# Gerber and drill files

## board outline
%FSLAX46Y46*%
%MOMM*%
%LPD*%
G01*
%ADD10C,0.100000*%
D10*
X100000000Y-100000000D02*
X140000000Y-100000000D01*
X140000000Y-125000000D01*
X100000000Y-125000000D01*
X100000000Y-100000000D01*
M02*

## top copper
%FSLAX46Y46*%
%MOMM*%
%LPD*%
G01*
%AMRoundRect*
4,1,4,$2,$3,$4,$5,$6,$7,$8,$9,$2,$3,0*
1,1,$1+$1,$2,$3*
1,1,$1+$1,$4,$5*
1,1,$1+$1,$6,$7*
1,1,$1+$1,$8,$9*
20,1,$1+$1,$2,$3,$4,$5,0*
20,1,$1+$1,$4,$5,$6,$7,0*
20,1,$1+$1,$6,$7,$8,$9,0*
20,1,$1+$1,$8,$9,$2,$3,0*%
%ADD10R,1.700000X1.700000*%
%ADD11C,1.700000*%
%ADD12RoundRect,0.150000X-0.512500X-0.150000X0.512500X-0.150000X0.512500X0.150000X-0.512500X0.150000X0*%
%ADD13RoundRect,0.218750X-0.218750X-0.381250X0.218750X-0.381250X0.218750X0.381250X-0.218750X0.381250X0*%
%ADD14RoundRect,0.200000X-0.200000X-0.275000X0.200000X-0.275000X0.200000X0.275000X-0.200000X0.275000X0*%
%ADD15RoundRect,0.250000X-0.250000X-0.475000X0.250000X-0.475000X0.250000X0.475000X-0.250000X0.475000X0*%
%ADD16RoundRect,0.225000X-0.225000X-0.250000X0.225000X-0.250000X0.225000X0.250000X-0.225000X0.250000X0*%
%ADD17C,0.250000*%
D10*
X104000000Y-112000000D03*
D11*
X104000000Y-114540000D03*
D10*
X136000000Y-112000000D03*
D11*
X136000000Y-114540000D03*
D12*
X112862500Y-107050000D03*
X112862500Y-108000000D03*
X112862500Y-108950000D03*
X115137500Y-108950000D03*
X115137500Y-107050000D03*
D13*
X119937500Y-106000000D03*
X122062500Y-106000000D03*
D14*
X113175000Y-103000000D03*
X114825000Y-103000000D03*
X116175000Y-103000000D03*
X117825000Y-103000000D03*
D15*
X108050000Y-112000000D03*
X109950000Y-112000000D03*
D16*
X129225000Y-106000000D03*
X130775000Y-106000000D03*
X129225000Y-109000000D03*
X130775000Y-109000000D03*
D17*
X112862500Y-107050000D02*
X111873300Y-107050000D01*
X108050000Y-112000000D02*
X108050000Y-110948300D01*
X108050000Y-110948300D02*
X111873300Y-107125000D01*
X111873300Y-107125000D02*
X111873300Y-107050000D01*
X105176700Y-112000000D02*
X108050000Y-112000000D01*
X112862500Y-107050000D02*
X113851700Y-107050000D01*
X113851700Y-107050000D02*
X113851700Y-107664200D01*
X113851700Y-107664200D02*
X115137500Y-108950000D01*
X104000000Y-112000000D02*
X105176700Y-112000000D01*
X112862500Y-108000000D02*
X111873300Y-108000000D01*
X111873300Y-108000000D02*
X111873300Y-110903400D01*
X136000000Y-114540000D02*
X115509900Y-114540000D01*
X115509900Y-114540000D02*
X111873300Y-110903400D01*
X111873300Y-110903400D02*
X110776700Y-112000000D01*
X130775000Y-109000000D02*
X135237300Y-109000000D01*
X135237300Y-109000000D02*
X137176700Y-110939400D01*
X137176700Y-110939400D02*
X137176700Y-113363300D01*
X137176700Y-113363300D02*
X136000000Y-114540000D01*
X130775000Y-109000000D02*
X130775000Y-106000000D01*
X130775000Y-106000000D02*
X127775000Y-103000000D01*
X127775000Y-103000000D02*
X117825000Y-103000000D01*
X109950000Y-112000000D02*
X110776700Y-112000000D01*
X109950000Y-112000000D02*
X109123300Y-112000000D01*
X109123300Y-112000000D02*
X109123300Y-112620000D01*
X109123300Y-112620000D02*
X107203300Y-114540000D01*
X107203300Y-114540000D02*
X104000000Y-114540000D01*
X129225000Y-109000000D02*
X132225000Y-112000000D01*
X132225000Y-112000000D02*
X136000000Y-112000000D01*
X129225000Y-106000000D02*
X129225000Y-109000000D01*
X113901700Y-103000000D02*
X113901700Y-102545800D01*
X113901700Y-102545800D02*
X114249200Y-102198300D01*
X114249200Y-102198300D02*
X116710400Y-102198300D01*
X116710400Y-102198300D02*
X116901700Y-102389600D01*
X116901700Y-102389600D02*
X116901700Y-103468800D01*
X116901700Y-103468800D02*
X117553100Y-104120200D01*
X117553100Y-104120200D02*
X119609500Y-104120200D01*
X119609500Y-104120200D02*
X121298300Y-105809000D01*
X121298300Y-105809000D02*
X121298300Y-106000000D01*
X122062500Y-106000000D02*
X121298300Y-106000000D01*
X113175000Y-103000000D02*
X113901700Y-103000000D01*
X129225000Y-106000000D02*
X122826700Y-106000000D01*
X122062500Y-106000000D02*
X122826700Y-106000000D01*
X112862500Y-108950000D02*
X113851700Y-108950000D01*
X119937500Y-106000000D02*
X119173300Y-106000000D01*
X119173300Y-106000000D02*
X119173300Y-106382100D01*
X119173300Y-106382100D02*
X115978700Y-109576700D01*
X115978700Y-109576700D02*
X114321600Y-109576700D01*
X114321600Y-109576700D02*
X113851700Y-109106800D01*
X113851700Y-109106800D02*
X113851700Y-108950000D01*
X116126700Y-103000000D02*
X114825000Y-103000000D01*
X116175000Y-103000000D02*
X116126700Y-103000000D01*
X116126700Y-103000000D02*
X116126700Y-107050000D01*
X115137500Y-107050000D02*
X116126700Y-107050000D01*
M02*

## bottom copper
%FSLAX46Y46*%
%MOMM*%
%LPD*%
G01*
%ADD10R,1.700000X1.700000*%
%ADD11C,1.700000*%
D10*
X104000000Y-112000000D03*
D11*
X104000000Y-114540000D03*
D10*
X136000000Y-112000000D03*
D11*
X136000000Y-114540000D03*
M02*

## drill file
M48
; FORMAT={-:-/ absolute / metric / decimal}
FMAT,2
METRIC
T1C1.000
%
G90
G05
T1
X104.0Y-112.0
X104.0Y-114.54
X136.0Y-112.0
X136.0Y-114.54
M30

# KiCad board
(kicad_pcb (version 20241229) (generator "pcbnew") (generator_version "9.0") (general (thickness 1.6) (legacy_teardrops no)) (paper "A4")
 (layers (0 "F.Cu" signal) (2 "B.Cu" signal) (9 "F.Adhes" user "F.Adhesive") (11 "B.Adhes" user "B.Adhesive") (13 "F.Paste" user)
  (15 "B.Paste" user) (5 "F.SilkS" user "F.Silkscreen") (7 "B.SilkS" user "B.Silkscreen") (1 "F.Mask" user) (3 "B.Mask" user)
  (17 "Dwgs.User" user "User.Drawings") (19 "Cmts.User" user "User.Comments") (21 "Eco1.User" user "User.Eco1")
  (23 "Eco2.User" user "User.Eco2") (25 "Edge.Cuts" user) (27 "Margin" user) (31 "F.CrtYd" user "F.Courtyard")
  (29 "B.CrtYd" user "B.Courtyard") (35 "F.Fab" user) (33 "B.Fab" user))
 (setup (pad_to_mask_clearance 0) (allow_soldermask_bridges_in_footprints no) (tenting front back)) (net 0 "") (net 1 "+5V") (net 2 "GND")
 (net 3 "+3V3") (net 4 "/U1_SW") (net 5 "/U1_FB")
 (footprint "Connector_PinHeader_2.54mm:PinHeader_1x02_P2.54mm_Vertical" (layer "F.Cu") (at 104 112)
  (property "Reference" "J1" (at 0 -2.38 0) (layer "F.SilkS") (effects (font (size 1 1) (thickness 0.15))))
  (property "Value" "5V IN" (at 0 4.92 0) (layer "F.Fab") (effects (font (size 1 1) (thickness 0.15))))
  (pad "1" thru_hole rect (at 0 0) (size 1.7 1.7) (drill 1) (layers "*.Cu" "*.Mask") (remove_unused_layers no) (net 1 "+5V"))
  (pad "2" thru_hole circle (at 0 2.54) (size 1.7 1.7) (drill 1) (layers "*.Cu" "*.Mask") (remove_unused_layers no) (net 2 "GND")))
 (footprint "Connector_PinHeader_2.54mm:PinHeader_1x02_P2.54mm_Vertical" (layer "F.Cu") (at 136 112)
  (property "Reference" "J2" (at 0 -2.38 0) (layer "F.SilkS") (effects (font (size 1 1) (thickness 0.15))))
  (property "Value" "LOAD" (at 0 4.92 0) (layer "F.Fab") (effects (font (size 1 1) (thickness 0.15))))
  (pad "1" thru_hole rect (at 0 0) (size 1.7 1.7) (drill 1) (layers "*.Cu" "*.Mask") (remove_unused_layers no) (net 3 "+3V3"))
  (pad "2" thru_hole circle (at 0 2.54) (size 1.7 1.7) (drill 1) (layers "*.Cu" "*.Mask") (remove_unused_layers no) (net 2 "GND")))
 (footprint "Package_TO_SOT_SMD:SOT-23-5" (layer "F.Cu") (at 114 108)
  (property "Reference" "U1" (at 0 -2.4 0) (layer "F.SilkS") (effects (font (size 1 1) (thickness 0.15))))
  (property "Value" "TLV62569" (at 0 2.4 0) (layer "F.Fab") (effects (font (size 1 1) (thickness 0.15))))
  (pad "1" smd roundrect (at -1.1375 -0.95) (size 1.325 0.6) (layers "F.Cu" "F.Mask" "F.Paste") (roundrect_rratio 0.25) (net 1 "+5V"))
  (pad "2" smd roundrect (at -1.1375 0) (size 1.325 0.6) (layers "F.Cu" "F.Mask" "F.Paste") (roundrect_rratio 0.25) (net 2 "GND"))
  (pad "3" smd roundrect (at -1.1375 0.95) (size 1.325 0.6) (layers "F.Cu" "F.Mask" "F.Paste") (roundrect_rratio 0.25) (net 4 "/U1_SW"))
  (pad "4" smd roundrect (at 1.1375 0.95) (size 1.325 0.6) (layers "F.Cu" "F.Mask" "F.Paste") (roundrect_rratio 0.25) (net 1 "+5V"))
  (pad "5" smd roundrect (at 1.1375 -0.95) (size 1.325 0.6) (layers "F.Cu" "F.Mask" "F.Paste") (roundrect_rratio 0.25) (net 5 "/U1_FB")))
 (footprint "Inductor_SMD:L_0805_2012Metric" (layer "F.Cu") (at 121 106)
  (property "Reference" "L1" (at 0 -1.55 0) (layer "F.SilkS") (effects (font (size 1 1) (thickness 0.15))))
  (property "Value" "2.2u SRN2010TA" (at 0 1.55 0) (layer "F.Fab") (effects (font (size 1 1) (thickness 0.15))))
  (pad "1" smd roundrect (at -1.0625 0) (size 0.875 1.2) (layers "F.Cu" "F.Mask" "F.Paste") (roundrect_rratio 0.25) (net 4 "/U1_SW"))
  (pad "2" smd roundrect (at 1.0625 0) (size 0.875 1.2) (layers "F.Cu" "F.Mask" "F.Paste") (roundrect_rratio 0.25) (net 3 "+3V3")))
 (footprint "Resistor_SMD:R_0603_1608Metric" (layer "F.Cu") (at 114 103)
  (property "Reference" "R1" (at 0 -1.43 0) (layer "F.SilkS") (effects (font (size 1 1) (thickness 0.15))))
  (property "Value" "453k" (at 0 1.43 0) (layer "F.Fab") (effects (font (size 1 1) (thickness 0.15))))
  (pad "1" smd roundrect (at -0.825 0) (size 0.8 0.95) (layers "F.Cu" "F.Mask" "F.Paste") (roundrect_rratio 0.25) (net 3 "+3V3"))
  (pad "2" smd roundrect (at 0.825 0) (size 0.8 0.95) (layers "F.Cu" "F.Mask" "F.Paste") (roundrect_rratio 0.25) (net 5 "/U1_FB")))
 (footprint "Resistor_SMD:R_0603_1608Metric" (layer "F.Cu") (at 117 103)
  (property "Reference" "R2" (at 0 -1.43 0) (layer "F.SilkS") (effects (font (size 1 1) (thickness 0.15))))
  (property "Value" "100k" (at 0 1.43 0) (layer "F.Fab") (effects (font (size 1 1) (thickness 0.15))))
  (pad "1" smd roundrect (at -0.825 0) (size 0.8 0.95) (layers "F.Cu" "F.Mask" "F.Paste") (roundrect_rratio 0.25) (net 5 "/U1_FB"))
  (pad "2" smd roundrect (at 0.825 0) (size 0.8 0.95) (layers "F.Cu" "F.Mask" "F.Paste") (roundrect_rratio 0.25) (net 2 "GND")))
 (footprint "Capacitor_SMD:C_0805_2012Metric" (layer "F.Cu") (at 109 112)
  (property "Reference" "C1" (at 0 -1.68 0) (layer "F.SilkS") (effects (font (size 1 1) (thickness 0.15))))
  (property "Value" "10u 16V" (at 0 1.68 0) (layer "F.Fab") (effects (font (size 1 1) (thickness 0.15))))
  (pad "1" smd roundrect (at -0.95 0) (size 1 1.45) (layers "F.Cu" "F.Mask" "F.Paste") (roundrect_rratio 0.25) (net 1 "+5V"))
  (pad "2" smd roundrect (at 0.95 0) (size 1 1.45) (layers "F.Cu" "F.Mask" "F.Paste") (roundrect_rratio 0.25) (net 2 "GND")))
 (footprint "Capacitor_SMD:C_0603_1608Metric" (layer "F.Cu") (at 130 106)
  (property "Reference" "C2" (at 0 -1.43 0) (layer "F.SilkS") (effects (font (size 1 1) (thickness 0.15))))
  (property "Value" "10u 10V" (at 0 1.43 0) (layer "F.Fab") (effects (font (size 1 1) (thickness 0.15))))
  (pad "1" smd roundrect (at -0.775 0) (size 0.9 0.95) (layers "F.Cu" "F.Mask" "F.Paste") (roundrect_rratio 0.25) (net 3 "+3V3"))
  (pad "2" smd roundrect (at 0.775 0) (size 0.9 0.95) (layers "F.Cu" "F.Mask" "F.Paste") (roundrect_rratio 0.25) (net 2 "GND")))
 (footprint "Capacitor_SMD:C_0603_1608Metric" (layer "F.Cu") (at 130 109)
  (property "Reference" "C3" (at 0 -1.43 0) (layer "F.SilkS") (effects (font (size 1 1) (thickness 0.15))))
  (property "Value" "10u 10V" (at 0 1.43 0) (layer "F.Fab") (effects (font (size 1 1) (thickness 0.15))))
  (pad "1" smd roundrect (at -0.775 0) (size 0.9 0.95) (layers "F.Cu" "F.Mask" "F.Paste") (roundrect_rratio 0.25) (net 3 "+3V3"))
  (pad "2" smd roundrect (at 0.775 0) (size 0.9 0.95) (layers "F.Cu" "F.Mask" "F.Paste") (roundrect_rratio 0.25) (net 2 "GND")))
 (gr_rect (start 100 100) (end 140 125) (stroke (width 0.1) (type default)) (fill no) (layer "Edge.Cuts"))
 (segment (start 112.8625 107.05) (end 111.8733 107.05) (width 0.25) (layer "F.Cu") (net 1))
 (segment (start 108.05 112) (end 108.05 110.9483) (width 0.25) (layer "F.Cu") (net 1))
 (segment (start 108.05 110.9483) (end 111.8733 107.125) (width 0.25) (layer "F.Cu") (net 1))
 (segment (start 111.8733 107.125) (end 111.8733 107.05) (width 0.25) (layer "F.Cu") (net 1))
 (segment (start 105.1767 112) (end 108.05 112) (width 0.25) (layer "F.Cu") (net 1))
 (segment (start 112.8625 107.05) (end 113.8517 107.05) (width 0.25) (layer "F.Cu") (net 1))
 (segment (start 113.8517 107.05) (end 113.8517 107.6642) (width 0.25) (layer "F.Cu") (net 1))
 (segment (start 113.8517 107.6642) (end 115.1375 108.95) (width 0.25) (layer "F.Cu") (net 1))
 (segment (start 104 112) (end 105.1767 112) (width 0.25) (layer "F.Cu") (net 1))
 (segment (start 112.8625 108) (end 111.8733 108) (width 0.25) (layer "F.Cu") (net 2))
 (segment (start 111.8733 108) (end 111.8733 110.9034) (width 0.25) (layer "F.Cu") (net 2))
 (segment (start 136 114.54) (end 115.5099 114.54) (width 0.25) (layer "F.Cu") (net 2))
 (segment (start 115.5099 114.54) (end 111.8733 110.9034) (width 0.25) (layer "F.Cu") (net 2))
 (segment (start 111.8733 110.9034) (end 110.7767 112) (width 0.25) (layer "F.Cu") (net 2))
 (segment (start 130.775 109) (end 135.2373 109) (width 0.25) (layer "F.Cu") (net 2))
 (segment (start 135.2373 109) (end 137.1767 110.9394) (width 0.25) (layer "F.Cu") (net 2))
 (segment (start 137.1767 110.9394) (end 137.1767 113.3633) (width 0.25) (layer "F.Cu") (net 2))
 (segment (start 137.1767 113.3633) (end 136 114.54) (width 0.25) (layer "F.Cu") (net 2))
 (segment (start 130.775 109) (end 130.775 106) (width 0.25) (layer "F.Cu") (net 2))
 (segment (start 130.775 106) (end 127.775 103) (width 0.25) (layer "F.Cu") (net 2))
 (segment (start 127.775 103) (end 117.825 103) (width 0.25) (layer "F.Cu") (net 2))
 (segment (start 109.95 112) (end 110.7767 112) (width 0.25) (layer "F.Cu") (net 2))
 (segment (start 109.95 112) (end 109.1233 112) (width 0.25) (layer "F.Cu") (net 2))
 (segment (start 109.1233 112) (end 109.1233 112.62) (width 0.25) (layer "F.Cu") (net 2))
 (segment (start 109.1233 112.62) (end 107.2033 114.54) (width 0.25) (layer "F.Cu") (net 2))
 (segment (start 107.2033 114.54) (end 104 114.54) (width 0.25) (layer "F.Cu") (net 2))
 (segment (start 129.225 109) (end 132.225 112) (width 0.25) (layer "F.Cu") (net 3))
 (segment (start 132.225 112) (end 136 112) (width 0.25) (layer "F.Cu") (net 3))
 (segment (start 129.225 106) (end 129.225 109) (width 0.25) (layer "F.Cu") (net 3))
 (segment (start 113.9017 103) (end 113.9017 102.5458) (width 0.25) (layer "F.Cu") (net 3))
 (segment (start 113.9017 102.5458) (end 114.2492 102.1983) (width 0.25) (layer "F.Cu") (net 3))
 (segment (start 114.2492 102.1983) (end 116.7104 102.1983) (width 0.25) (layer "F.Cu") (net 3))
 (segment (start 116.7104 102.1983) (end 116.9017 102.3896) (width 0.25) (layer "F.Cu") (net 3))
 (segment (start 116.9017 102.3896) (end 116.9017 103.4688) (width 0.25) (layer "F.Cu") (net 3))
 (segment (start 116.9017 103.4688) (end 117.5531 104.1202) (width 0.25) (layer "F.Cu") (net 3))
 (segment (start 117.5531 104.1202) (end 119.6095 104.1202) (width 0.25) (layer "F.Cu") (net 3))
 (segment (start 119.6095 104.1202) (end 121.2983 105.809) (width 0.25) (layer "F.Cu") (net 3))
 (segment (start 121.2983 105.809) (end 121.2983 106) (width 0.25) (layer "F.Cu") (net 3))
 (segment (start 122.0625 106) (end 121.2983 106) (width 0.25) (layer "F.Cu") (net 3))
 (segment (start 113.175 103) (end 113.9017 103) (width 0.25) (layer "F.Cu") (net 3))
 (segment (start 129.225 106) (end 122.8267 106) (width 0.25) (layer "F.Cu") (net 3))
 (segment (start 122.0625 106) (end 122.8267 106) (width 0.25) (layer "F.Cu") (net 3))
 (segment (start 112.8625 108.95) (end 113.8517 108.95) (width 0.25) (layer "F.Cu") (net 4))
 (segment (start 119.9375 106) (end 119.1733 106) (width 0.25) (layer "F.Cu") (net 4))
 (segment (start 119.1733 106) (end 119.1733 106.3821) (width 0.25) (layer "F.Cu") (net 4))
 (segment (start 119.1733 106.3821) (end 115.9787 109.5767) (width 0.25) (layer "F.Cu") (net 4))
 (segment (start 115.9787 109.5767) (end 114.3216 109.5767) (width 0.25) (layer "F.Cu") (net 4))
 (segment (start 114.3216 109.5767) (end 113.8517 109.1068) (width 0.25) (layer "F.Cu") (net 4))
 (segment (start 113.8517 109.1068) (end 113.8517 108.95) (width 0.25) (layer "F.Cu") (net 4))
 (segment (start 116.1267 103) (end 114.825 103) (width 0.25) (layer "F.Cu") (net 5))
 (segment (start 116.175 103) (end 116.1267 103) (width 0.25) (layer "F.Cu") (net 5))
 (segment (start 116.1267 103) (end 116.1267 107.05) (width 0.25) (layer "F.Cu") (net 5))
 (segment (start 115.1375 107.05) (end 116.1267 107.05) (width 0.25) (layer "F.Cu") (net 5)))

